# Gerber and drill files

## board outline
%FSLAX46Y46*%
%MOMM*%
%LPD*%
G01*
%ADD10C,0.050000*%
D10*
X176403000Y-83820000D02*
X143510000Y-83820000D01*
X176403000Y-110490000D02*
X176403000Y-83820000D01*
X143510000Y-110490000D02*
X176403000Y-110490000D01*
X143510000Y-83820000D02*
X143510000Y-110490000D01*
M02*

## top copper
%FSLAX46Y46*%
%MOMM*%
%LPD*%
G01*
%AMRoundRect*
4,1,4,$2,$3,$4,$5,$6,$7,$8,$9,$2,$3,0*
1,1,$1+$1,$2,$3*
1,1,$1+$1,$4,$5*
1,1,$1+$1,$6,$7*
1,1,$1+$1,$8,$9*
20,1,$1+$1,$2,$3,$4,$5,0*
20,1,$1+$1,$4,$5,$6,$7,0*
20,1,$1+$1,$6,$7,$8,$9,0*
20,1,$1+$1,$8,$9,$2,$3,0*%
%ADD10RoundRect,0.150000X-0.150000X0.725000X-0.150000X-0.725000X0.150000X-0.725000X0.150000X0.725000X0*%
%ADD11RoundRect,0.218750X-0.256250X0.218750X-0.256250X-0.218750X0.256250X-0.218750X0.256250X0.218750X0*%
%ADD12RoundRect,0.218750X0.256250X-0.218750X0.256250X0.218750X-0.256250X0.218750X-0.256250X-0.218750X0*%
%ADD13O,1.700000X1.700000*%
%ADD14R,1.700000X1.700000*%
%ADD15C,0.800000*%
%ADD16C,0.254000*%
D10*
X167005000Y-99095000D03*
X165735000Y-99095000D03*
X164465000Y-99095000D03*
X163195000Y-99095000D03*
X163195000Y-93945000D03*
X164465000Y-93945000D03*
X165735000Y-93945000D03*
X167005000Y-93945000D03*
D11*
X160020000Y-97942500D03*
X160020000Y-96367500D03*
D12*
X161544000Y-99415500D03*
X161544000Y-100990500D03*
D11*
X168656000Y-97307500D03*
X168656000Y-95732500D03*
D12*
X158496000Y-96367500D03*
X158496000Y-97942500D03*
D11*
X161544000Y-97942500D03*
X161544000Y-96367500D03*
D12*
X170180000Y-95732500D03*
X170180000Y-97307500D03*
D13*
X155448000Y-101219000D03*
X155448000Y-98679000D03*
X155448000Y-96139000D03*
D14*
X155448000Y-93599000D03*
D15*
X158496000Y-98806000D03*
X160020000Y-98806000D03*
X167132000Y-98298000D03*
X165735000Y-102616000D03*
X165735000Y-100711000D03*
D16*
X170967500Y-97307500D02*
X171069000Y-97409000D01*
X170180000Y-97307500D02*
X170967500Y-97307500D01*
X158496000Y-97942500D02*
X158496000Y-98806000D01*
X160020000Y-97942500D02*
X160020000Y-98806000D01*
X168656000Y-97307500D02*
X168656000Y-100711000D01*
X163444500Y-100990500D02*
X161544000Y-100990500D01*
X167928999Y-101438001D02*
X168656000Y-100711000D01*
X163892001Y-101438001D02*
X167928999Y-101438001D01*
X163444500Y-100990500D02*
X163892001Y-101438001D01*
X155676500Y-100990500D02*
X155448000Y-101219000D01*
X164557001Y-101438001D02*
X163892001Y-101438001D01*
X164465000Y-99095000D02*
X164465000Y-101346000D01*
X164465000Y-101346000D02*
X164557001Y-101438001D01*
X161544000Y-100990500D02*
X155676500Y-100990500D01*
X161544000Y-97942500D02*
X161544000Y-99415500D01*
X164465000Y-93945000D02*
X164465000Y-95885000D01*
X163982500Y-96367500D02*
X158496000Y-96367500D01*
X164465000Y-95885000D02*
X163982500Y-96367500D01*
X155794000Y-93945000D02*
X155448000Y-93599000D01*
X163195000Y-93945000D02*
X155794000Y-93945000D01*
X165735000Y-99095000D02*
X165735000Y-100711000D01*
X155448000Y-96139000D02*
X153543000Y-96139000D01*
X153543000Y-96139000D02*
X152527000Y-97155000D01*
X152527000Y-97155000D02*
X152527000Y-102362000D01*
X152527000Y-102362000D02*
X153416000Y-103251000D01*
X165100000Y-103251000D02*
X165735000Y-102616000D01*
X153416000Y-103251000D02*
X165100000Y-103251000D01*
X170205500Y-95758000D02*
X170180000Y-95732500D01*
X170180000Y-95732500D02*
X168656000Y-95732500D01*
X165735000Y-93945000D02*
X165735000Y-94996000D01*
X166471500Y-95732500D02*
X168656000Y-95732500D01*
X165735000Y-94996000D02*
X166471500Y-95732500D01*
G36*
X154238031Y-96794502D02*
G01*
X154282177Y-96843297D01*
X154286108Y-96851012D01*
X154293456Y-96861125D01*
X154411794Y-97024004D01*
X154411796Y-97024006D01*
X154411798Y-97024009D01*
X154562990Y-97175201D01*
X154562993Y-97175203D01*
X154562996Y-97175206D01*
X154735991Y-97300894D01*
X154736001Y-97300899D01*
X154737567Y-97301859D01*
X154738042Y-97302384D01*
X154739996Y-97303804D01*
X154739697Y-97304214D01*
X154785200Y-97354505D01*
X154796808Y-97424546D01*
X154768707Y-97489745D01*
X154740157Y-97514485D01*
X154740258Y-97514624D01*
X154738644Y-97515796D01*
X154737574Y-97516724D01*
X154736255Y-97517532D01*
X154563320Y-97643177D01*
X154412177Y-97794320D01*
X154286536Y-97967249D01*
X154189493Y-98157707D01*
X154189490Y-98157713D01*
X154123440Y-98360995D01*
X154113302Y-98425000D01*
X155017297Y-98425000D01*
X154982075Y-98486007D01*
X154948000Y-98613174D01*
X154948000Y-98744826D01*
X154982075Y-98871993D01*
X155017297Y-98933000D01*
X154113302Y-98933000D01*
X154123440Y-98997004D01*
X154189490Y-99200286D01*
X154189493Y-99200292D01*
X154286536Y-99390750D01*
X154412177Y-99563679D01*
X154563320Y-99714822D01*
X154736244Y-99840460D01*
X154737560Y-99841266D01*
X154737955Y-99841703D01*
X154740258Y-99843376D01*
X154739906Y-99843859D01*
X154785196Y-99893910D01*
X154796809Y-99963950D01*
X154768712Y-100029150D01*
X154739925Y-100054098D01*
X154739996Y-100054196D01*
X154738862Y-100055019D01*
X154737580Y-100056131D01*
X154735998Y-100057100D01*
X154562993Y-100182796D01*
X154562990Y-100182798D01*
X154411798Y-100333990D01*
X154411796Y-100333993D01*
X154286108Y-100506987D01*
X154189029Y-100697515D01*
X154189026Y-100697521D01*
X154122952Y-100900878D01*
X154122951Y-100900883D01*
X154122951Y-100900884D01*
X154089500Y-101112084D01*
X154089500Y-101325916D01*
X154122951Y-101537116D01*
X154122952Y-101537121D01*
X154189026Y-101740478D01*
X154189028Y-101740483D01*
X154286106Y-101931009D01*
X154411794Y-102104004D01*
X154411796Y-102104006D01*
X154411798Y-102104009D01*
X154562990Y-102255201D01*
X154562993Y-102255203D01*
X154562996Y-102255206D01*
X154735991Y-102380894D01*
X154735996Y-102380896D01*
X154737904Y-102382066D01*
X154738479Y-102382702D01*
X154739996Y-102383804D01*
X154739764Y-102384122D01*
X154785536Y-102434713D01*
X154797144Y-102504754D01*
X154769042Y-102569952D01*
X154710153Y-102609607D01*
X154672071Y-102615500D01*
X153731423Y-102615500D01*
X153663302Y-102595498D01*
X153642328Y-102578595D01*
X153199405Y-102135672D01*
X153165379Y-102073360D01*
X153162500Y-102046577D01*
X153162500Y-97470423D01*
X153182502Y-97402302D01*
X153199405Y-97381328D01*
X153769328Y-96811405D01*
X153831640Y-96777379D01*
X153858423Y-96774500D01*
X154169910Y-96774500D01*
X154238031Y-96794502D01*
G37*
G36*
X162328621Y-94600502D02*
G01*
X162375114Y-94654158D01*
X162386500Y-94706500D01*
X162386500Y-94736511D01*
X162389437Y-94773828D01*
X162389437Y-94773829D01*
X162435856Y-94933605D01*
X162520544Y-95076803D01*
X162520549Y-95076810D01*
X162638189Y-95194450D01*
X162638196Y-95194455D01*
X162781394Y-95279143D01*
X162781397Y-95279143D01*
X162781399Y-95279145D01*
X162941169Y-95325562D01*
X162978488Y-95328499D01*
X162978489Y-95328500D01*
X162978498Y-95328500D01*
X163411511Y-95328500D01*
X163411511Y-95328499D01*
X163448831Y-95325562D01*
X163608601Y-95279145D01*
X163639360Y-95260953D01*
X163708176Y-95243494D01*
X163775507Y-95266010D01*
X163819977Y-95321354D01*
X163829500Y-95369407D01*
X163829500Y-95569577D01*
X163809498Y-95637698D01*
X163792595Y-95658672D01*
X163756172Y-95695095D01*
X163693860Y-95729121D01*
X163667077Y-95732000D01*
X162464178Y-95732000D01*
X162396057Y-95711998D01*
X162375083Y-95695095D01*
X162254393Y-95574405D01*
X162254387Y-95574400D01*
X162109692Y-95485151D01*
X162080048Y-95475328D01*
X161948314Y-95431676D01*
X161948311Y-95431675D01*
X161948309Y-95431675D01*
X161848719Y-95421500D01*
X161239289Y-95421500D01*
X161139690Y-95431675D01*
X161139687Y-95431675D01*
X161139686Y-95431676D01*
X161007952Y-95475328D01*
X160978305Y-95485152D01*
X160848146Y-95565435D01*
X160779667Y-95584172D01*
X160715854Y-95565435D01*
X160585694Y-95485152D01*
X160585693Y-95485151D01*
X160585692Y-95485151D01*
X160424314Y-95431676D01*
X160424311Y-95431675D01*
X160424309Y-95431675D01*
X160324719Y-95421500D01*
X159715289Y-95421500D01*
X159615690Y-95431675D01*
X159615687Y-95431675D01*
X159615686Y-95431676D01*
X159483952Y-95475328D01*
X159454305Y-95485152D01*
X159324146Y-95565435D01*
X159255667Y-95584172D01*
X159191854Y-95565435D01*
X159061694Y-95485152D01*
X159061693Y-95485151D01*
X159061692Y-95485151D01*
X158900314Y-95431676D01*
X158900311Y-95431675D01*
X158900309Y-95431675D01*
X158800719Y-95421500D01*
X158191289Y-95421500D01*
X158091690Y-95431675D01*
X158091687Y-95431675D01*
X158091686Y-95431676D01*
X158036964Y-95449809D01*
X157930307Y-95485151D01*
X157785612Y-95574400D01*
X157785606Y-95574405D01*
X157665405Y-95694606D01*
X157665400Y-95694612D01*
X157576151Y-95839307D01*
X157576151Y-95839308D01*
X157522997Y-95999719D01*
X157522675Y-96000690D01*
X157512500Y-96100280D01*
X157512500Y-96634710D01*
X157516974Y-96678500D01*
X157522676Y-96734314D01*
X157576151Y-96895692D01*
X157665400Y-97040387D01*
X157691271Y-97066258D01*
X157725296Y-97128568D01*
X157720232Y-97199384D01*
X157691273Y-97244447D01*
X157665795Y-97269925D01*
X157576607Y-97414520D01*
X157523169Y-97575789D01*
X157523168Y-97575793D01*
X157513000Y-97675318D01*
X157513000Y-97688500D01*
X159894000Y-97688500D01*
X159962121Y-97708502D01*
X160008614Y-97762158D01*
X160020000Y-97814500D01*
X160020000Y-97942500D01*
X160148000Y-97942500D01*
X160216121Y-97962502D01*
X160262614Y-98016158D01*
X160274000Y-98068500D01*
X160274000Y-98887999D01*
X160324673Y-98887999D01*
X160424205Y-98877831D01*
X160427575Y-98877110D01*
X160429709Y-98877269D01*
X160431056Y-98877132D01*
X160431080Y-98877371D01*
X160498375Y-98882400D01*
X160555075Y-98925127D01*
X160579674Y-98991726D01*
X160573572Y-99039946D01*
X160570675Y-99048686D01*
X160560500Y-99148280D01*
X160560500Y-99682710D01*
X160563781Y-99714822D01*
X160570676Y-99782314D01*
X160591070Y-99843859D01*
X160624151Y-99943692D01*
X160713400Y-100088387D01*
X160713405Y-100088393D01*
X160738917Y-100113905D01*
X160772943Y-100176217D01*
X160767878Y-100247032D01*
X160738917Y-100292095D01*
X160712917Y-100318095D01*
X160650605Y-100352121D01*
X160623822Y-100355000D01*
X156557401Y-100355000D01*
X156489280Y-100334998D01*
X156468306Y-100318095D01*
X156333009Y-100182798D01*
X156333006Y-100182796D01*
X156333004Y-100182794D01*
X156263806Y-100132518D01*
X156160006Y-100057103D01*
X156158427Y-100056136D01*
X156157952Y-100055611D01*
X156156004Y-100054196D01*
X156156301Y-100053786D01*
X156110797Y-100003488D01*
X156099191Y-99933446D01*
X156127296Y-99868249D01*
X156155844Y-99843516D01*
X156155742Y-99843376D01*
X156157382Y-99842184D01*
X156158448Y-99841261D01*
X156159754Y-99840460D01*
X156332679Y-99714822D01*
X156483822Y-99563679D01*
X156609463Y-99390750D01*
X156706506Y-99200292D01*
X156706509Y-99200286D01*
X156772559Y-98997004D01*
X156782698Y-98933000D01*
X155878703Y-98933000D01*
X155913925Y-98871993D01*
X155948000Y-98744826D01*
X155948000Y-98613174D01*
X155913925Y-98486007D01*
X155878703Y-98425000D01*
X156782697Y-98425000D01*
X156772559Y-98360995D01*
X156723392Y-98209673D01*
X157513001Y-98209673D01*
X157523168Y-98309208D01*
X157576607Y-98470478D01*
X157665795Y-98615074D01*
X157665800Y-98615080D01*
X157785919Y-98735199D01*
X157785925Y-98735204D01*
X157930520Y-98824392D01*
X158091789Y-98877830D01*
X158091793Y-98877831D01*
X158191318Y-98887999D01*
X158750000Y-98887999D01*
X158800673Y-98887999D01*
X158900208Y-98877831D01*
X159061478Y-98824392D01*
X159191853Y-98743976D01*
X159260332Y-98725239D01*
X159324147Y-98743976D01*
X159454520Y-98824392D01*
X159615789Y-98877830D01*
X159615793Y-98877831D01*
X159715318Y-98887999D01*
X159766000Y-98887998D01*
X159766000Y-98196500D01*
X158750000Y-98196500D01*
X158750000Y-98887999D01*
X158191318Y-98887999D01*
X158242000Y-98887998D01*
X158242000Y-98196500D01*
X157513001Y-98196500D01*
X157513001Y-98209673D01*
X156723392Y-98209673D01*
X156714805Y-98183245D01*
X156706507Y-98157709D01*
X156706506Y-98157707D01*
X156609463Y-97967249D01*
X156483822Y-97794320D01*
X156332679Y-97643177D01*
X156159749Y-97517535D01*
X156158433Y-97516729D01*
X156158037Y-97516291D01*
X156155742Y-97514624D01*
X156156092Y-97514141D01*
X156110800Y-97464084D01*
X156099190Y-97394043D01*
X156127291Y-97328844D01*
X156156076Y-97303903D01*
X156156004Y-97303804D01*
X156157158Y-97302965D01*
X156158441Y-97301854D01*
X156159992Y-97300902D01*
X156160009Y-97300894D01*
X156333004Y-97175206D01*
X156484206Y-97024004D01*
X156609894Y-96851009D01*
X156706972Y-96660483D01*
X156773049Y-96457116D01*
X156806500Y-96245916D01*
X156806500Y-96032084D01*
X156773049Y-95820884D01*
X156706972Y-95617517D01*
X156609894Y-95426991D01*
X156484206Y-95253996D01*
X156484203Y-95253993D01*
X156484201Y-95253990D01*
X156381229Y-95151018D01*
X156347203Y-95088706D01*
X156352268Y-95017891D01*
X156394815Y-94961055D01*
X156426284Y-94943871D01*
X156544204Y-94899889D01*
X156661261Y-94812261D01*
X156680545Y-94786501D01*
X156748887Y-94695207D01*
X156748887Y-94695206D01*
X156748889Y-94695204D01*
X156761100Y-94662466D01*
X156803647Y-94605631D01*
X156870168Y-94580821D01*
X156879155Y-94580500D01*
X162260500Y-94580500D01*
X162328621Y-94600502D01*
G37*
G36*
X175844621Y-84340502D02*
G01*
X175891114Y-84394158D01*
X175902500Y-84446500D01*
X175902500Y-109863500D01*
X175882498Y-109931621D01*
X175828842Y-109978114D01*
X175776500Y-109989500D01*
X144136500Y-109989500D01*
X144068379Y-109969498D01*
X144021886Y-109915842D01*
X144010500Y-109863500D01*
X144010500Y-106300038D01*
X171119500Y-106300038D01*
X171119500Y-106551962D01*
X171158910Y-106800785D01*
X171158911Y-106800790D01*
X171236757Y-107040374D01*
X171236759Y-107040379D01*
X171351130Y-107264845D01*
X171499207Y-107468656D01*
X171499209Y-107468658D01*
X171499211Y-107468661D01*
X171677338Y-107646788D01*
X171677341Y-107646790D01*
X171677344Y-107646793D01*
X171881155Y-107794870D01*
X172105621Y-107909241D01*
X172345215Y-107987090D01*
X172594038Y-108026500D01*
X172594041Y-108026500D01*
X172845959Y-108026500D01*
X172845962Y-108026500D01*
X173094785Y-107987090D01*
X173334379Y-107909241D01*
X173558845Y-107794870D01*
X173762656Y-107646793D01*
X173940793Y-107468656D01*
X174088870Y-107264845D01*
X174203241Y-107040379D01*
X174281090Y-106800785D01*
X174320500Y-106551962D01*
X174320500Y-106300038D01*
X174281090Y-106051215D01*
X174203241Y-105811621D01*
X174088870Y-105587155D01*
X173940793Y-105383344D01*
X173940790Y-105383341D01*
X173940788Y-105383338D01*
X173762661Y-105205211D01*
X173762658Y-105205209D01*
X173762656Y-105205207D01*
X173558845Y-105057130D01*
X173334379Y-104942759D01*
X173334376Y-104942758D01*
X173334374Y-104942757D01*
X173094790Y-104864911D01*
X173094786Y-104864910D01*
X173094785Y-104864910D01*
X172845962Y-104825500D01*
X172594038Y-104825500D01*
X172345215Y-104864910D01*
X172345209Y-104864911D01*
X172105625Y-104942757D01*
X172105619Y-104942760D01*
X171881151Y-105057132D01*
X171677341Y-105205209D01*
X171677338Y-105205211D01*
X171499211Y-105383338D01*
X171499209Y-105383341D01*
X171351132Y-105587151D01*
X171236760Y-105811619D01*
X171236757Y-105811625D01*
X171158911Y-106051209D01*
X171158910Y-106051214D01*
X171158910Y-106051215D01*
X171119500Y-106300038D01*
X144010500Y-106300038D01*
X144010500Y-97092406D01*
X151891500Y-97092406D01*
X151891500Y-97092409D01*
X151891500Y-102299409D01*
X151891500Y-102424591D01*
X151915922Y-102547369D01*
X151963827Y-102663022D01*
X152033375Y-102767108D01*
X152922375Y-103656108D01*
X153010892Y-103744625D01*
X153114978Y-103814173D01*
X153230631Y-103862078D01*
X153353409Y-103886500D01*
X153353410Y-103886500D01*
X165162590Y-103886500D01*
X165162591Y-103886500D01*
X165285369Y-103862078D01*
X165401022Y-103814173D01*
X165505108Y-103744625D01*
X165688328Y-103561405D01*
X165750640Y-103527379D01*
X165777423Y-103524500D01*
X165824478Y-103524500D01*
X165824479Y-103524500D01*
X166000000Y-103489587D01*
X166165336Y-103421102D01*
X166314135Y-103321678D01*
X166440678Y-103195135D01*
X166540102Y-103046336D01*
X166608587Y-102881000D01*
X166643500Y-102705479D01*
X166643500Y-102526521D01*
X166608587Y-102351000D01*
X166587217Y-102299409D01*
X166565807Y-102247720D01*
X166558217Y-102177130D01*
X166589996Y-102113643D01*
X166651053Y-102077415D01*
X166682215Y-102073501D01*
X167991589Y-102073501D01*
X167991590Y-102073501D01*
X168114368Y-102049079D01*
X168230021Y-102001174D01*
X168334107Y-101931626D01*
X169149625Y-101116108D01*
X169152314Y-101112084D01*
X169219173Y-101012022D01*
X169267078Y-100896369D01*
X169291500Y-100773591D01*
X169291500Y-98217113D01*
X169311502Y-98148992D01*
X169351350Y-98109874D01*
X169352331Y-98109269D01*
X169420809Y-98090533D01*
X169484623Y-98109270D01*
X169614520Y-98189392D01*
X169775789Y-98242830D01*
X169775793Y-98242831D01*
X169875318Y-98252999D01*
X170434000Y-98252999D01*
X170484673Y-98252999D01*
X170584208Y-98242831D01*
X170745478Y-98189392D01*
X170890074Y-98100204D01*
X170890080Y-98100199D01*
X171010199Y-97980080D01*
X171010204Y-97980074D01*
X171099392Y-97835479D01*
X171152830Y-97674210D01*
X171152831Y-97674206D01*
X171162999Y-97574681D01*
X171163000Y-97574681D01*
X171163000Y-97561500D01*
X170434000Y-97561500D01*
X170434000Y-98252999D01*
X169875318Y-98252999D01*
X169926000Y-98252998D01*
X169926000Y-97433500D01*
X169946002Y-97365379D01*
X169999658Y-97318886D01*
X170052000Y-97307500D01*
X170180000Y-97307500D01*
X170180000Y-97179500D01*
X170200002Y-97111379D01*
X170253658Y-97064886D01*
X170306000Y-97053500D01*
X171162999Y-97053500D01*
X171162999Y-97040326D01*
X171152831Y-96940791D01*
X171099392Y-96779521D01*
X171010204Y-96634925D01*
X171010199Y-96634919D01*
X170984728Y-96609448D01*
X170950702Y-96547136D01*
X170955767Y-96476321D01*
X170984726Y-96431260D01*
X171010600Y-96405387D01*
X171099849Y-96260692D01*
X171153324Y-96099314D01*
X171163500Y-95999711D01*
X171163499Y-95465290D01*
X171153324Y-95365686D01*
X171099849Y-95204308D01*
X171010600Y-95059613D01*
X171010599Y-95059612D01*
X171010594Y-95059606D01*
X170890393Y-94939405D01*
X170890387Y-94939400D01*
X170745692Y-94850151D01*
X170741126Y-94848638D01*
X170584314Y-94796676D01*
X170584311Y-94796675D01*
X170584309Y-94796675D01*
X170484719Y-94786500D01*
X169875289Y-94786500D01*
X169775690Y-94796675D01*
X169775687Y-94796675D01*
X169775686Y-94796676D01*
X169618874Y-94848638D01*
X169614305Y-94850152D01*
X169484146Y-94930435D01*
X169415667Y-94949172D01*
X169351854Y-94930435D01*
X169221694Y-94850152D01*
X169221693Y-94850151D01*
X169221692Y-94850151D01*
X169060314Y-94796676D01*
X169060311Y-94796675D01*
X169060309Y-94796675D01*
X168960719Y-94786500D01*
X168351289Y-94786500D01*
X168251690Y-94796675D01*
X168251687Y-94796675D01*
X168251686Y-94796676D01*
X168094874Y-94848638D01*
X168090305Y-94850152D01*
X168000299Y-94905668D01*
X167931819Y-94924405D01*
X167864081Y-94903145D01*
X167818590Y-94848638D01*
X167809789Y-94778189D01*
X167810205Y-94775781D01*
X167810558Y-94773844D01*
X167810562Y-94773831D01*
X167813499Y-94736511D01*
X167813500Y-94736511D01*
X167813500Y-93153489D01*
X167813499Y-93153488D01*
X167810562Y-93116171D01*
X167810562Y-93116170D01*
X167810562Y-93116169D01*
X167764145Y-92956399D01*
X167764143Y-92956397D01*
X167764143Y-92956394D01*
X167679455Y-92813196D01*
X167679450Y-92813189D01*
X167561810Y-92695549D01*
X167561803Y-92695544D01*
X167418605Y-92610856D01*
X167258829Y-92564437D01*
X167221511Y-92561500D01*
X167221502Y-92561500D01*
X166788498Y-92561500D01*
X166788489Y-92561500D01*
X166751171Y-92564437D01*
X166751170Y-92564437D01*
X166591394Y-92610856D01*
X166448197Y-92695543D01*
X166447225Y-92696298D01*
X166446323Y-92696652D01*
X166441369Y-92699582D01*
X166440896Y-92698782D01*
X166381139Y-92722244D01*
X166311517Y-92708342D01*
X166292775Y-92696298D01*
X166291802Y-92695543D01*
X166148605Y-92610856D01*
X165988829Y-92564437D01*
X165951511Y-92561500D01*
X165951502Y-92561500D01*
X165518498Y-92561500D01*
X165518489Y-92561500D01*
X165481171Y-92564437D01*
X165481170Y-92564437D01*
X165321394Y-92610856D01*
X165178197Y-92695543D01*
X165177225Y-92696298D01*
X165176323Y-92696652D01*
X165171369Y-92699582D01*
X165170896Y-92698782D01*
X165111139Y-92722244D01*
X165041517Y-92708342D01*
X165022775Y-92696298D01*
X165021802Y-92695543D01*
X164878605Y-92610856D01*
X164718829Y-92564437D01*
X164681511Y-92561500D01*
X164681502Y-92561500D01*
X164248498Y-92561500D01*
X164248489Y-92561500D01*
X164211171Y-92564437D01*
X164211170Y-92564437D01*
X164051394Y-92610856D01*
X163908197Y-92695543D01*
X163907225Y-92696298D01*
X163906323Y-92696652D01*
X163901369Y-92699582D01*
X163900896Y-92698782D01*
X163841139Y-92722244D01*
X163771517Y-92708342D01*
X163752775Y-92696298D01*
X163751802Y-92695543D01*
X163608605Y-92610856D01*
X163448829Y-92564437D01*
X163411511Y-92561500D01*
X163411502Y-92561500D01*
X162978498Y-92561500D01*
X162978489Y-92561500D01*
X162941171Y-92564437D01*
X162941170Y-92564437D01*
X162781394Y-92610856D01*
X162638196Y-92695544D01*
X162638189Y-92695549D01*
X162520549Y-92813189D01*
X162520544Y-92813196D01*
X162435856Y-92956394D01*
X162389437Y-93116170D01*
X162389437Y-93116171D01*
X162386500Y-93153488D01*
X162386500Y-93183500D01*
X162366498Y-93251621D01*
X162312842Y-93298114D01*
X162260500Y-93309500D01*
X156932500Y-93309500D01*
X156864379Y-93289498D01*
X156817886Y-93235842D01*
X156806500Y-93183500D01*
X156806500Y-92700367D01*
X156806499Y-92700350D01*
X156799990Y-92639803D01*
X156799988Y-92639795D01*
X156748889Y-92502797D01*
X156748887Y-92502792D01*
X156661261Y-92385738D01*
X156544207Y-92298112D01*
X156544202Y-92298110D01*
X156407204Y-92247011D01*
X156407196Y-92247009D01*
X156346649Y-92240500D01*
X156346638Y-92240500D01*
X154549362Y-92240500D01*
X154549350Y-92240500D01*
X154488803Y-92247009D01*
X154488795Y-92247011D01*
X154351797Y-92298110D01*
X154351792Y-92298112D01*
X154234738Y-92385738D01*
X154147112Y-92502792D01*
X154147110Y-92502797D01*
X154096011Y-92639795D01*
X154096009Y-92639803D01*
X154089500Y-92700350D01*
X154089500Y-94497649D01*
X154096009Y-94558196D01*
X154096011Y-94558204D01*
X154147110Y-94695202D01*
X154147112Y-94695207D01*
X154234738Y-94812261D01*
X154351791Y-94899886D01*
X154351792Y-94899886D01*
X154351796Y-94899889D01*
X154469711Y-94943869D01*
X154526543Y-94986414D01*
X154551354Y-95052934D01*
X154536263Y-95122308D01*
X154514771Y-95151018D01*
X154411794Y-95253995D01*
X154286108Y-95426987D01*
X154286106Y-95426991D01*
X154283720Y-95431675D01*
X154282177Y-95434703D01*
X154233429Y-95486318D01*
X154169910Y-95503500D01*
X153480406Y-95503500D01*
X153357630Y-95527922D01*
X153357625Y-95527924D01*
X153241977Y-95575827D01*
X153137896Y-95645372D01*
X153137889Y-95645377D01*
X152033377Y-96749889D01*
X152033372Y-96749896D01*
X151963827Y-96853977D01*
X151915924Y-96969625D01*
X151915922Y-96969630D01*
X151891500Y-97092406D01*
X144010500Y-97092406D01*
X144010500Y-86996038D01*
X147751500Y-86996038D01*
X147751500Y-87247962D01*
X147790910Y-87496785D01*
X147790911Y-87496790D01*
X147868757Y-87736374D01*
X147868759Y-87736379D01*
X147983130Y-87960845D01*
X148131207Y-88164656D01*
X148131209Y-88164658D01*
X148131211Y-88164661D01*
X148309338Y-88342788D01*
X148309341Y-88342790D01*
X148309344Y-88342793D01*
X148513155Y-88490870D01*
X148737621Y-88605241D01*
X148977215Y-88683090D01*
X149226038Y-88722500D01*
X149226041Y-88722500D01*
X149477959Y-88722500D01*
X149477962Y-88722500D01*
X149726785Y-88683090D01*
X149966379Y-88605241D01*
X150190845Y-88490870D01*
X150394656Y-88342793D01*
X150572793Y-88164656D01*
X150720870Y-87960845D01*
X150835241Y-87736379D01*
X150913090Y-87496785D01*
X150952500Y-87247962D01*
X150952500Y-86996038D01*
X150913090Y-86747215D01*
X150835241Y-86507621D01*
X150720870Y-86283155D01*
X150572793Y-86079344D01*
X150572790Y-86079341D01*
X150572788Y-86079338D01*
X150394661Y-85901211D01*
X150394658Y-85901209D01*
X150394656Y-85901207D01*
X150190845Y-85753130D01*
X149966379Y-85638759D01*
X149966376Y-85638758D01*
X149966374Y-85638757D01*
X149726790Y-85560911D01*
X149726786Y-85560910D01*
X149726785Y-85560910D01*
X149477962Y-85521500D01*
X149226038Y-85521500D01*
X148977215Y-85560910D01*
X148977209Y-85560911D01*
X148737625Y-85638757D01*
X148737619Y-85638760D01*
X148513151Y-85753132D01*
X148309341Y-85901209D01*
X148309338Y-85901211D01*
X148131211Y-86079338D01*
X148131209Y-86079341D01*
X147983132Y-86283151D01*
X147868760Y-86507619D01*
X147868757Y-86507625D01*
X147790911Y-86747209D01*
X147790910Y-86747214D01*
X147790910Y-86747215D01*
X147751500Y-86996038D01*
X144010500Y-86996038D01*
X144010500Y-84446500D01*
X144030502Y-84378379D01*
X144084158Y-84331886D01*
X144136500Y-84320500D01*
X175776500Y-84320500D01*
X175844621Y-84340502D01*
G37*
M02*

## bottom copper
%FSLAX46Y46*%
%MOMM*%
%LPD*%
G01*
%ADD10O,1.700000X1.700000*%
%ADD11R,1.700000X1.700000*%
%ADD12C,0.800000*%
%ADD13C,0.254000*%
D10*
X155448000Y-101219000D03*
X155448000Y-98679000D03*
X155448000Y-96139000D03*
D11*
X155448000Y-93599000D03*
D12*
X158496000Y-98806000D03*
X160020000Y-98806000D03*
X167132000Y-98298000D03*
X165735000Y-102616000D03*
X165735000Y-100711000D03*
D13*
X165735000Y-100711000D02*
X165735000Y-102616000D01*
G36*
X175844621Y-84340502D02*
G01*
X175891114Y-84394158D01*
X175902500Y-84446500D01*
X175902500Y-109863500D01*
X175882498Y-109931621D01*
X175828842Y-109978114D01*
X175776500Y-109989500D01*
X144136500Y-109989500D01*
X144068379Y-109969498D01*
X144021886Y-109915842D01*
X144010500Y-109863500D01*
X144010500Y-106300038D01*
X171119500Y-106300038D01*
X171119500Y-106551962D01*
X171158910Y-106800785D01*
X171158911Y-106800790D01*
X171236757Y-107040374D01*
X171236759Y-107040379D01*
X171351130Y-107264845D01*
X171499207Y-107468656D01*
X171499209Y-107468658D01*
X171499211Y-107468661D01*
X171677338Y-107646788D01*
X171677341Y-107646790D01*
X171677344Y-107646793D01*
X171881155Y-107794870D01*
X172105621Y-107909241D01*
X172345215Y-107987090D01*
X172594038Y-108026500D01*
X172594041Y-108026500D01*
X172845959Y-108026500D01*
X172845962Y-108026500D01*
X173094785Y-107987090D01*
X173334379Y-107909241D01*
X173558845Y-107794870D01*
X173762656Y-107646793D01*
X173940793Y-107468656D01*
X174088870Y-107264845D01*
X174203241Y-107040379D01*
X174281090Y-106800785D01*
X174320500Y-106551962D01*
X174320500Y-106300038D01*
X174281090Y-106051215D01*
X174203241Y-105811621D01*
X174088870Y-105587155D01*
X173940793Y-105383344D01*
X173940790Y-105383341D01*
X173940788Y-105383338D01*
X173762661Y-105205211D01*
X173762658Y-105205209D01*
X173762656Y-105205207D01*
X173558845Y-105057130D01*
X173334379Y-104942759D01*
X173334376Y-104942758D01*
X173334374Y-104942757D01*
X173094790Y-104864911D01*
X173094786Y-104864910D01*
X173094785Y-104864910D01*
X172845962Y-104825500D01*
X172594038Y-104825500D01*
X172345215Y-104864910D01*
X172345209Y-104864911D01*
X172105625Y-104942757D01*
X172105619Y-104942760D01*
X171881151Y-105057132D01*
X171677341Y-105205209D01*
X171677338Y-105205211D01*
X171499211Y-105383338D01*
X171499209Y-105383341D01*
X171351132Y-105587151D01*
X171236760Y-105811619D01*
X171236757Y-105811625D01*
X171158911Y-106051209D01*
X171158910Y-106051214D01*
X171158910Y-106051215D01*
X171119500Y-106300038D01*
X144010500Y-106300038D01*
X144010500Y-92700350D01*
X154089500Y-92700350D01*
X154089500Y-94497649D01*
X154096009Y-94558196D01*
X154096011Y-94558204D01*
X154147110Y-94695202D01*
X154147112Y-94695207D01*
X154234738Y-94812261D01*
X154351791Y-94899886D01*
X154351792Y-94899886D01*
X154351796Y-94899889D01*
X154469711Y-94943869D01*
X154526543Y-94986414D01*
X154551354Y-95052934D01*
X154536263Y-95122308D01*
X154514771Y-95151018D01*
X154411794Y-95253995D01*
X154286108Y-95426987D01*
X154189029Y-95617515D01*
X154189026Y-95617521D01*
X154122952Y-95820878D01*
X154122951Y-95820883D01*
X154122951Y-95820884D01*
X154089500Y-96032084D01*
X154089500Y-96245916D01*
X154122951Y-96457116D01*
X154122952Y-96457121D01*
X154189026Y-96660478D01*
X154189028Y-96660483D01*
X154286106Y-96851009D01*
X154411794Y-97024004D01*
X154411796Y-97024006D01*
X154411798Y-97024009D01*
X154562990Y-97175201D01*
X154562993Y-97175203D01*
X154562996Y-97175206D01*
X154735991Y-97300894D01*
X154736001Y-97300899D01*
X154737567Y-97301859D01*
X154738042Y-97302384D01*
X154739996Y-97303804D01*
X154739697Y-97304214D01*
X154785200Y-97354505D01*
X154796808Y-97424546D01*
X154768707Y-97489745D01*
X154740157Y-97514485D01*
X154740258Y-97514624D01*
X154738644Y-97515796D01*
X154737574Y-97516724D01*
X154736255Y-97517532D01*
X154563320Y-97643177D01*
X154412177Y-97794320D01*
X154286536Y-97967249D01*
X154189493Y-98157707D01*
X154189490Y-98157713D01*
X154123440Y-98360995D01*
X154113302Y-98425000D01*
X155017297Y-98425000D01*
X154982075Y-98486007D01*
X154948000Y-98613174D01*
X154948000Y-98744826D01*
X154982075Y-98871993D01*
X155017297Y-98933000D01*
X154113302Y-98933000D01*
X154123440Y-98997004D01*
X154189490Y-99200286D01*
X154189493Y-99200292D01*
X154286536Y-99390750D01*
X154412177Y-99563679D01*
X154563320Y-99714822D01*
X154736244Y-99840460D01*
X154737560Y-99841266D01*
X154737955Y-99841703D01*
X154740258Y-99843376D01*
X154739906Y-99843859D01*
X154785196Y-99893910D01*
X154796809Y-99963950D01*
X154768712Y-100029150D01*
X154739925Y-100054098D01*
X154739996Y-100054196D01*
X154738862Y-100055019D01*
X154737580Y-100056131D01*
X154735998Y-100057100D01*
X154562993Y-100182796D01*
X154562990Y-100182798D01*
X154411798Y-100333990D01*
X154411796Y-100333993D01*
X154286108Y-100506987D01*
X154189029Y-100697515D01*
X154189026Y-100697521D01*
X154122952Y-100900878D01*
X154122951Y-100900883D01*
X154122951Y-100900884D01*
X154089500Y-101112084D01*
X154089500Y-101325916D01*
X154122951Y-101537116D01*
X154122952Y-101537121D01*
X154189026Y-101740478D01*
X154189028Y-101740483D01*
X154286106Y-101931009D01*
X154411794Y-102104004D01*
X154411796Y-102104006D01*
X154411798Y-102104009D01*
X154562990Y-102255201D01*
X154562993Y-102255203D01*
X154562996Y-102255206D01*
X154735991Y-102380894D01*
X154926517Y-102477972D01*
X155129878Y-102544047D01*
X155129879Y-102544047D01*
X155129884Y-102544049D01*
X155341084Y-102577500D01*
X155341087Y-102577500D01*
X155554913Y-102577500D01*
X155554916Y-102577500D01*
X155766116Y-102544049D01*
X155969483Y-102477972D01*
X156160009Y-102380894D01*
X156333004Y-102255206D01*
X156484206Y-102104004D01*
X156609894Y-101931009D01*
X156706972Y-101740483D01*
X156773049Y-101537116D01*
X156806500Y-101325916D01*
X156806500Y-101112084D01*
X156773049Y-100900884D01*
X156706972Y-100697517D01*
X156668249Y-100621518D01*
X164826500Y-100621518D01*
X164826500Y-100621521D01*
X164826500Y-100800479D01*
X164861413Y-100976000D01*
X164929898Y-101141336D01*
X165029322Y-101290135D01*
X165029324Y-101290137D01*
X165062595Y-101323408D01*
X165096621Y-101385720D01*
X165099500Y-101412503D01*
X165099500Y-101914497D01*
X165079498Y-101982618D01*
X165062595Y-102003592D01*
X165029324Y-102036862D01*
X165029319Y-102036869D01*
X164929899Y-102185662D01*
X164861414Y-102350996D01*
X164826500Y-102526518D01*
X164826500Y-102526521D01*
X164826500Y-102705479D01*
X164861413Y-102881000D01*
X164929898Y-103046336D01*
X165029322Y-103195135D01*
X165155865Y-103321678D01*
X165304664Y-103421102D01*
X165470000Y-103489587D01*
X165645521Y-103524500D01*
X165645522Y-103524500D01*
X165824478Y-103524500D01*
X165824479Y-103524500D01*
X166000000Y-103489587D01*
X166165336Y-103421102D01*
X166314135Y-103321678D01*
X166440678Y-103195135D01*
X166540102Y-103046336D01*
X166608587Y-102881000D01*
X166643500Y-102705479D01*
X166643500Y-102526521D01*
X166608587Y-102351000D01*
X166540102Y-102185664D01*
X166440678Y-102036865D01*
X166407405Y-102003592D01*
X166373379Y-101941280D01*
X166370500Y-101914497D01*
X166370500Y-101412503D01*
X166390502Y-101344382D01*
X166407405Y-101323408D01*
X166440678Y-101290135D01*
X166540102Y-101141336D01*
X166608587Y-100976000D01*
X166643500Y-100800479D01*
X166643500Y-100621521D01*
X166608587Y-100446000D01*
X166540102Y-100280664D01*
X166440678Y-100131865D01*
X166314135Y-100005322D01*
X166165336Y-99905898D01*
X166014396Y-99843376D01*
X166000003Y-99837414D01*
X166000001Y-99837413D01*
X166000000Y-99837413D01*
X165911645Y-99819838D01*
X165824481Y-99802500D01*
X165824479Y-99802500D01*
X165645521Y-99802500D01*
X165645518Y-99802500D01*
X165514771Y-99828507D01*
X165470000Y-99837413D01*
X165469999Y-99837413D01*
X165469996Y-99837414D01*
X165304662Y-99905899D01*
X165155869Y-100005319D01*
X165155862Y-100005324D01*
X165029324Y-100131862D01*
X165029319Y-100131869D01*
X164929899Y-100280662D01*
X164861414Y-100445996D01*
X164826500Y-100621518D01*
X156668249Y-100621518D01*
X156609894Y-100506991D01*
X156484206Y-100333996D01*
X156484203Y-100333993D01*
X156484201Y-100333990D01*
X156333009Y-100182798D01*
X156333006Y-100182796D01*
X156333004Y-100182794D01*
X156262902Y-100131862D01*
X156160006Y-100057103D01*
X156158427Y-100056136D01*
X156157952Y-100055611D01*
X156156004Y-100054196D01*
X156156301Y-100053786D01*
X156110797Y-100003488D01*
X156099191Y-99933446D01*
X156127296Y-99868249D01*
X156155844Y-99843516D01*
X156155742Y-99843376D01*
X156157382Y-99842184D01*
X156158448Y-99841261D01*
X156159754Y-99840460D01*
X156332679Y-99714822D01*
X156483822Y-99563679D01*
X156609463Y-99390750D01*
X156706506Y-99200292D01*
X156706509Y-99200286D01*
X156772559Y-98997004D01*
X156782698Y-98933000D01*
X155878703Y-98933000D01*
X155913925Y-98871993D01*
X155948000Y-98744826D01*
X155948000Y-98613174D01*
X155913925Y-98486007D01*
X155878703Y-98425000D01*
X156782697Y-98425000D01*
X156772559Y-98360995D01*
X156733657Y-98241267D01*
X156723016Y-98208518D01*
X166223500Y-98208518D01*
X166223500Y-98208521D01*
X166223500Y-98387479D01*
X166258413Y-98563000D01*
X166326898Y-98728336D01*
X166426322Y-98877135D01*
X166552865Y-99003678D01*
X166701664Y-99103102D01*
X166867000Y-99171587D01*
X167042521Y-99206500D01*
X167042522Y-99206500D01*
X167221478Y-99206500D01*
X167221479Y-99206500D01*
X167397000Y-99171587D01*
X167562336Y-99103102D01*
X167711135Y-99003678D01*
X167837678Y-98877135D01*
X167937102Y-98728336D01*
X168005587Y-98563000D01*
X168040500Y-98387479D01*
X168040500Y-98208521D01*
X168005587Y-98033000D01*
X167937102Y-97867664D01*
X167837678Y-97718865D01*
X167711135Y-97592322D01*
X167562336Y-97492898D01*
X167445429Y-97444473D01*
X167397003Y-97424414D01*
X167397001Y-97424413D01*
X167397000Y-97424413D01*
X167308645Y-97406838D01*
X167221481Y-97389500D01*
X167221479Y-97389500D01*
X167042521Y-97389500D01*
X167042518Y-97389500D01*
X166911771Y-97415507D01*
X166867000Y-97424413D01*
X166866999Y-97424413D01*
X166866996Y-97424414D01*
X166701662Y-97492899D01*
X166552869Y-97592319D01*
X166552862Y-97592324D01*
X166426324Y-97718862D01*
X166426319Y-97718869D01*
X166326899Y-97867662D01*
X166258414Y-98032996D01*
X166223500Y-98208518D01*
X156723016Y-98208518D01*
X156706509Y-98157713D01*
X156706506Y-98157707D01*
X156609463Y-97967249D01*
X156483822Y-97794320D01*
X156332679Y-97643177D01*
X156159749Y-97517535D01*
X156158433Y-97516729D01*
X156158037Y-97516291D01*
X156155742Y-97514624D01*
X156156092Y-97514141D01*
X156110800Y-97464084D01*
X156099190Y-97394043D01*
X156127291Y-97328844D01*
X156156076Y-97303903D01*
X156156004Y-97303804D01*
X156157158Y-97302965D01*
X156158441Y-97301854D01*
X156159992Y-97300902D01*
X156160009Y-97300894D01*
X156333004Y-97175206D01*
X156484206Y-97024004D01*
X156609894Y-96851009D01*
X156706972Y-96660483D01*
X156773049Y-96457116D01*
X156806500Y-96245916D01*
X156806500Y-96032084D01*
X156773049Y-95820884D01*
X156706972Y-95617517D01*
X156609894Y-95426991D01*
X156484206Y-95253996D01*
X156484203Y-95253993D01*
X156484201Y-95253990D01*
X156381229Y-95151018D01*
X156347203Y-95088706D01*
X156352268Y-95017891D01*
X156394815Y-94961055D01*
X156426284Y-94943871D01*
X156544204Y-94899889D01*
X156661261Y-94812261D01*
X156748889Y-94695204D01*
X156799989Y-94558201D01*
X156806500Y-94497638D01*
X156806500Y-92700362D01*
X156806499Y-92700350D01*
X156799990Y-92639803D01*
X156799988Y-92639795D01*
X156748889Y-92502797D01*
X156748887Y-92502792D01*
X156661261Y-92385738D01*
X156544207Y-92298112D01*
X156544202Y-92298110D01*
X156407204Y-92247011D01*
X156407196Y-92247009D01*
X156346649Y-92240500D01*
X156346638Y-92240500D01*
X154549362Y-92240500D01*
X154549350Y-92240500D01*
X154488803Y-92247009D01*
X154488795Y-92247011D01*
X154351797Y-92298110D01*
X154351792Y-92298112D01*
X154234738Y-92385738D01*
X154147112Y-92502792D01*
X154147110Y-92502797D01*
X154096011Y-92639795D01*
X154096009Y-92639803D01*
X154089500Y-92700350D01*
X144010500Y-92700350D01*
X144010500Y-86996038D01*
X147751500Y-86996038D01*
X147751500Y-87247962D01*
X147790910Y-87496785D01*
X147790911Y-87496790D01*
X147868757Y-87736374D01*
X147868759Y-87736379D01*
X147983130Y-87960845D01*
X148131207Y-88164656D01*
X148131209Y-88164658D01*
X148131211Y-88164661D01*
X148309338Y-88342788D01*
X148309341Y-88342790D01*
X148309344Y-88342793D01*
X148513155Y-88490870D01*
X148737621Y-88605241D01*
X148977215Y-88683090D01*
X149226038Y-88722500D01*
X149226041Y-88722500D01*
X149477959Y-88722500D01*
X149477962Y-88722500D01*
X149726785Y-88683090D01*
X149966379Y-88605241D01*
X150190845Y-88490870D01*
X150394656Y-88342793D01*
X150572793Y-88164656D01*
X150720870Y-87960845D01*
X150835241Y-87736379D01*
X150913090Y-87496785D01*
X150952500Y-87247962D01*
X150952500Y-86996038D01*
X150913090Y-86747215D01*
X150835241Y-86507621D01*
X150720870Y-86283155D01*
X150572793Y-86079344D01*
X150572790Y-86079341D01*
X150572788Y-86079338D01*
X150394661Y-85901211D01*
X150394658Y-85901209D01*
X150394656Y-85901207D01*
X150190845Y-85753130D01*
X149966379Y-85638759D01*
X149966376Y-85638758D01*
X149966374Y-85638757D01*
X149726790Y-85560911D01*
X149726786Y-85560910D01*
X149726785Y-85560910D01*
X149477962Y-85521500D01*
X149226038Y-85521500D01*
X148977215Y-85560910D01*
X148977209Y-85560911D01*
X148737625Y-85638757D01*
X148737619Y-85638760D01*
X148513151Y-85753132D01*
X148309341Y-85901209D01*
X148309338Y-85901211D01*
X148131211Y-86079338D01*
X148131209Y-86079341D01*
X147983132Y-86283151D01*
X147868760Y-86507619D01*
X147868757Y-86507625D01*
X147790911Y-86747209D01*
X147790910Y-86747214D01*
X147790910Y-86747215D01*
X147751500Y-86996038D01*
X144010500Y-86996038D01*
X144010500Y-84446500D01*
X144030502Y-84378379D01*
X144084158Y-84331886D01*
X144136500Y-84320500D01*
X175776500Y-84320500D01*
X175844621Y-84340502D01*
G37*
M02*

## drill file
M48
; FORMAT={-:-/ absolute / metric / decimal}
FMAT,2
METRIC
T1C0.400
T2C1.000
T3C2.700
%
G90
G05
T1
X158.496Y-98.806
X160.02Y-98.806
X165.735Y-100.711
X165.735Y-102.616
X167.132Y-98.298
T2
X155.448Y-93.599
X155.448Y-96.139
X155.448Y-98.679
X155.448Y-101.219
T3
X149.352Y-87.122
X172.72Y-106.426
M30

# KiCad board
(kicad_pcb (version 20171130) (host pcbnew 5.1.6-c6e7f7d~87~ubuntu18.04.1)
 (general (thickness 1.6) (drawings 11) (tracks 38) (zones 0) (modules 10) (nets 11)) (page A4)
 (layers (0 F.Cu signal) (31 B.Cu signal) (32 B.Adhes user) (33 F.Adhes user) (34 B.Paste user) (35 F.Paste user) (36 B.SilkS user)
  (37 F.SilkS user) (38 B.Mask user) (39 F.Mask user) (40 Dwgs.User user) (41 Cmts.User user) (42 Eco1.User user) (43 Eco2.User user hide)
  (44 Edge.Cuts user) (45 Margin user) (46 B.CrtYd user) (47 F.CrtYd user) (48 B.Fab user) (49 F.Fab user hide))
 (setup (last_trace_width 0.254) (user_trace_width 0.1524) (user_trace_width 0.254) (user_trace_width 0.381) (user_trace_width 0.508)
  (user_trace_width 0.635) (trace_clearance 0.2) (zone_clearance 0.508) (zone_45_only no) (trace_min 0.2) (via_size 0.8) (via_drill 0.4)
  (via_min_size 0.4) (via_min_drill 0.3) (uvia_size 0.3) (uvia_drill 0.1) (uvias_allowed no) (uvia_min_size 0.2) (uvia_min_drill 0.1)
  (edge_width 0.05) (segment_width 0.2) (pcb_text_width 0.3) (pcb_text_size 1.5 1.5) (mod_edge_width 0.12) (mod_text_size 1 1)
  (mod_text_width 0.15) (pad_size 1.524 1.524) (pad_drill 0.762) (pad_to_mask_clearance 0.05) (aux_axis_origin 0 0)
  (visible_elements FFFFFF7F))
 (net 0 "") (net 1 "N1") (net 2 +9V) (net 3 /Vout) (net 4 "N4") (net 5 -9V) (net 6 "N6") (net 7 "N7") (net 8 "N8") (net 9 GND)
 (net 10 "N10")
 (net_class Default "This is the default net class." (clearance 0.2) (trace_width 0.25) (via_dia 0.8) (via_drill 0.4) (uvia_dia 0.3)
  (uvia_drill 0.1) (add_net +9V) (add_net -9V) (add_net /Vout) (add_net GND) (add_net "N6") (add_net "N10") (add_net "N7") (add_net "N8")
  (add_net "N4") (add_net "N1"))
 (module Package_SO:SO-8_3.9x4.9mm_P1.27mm (layer F.Cu) (at 165.1 96.52 270)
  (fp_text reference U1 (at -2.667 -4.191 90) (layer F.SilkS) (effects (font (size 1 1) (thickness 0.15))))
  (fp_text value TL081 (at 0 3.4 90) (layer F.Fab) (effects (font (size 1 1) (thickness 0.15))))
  (pad 8 smd roundrect (at 2.575 -1.905 270) (size 1.75 0.6) (layers F.Cu F.Paste F.Mask) (roundrect_rratio 0.25) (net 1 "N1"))
  (pad 7 smd roundrect (at 2.575 -0.635 270) (size 1.75 0.6) (layers F.Cu F.Paste F.Mask) (roundrect_rratio 0.25) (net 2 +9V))
  (pad 6 smd roundrect (at 2.575 0.635 270) (size 1.75 0.6) (layers F.Cu F.Paste F.Mask) (roundrect_rratio 0.25) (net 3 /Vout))
  (pad 5 smd roundrect (at 2.575 1.905 270) (size 1.75 0.6) (layers F.Cu F.Paste F.Mask) (roundrect_rratio 0.25) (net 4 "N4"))
  (pad 4 smd roundrect (at -2.575 1.905 270) (size 1.75 0.6) (layers F.Cu F.Paste F.Mask) (roundrect_rratio 0.25) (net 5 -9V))
  (pad 3 smd roundrect (at -2.575 0.635 270) (size 1.75 0.6) (layers F.Cu F.Paste F.Mask) (roundrect_rratio 0.25) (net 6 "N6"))
  (pad 2 smd roundrect (at -2.575 -0.635 270) (size 1.75 0.6) (layers F.Cu F.Paste F.Mask) (roundrect_rratio 0.25) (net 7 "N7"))
  (pad 1 smd roundrect (at -2.575 -1.905 270) (size 1.75 0.6) (layers F.Cu F.Paste F.Mask) (roundrect_rratio 0.25) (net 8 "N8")))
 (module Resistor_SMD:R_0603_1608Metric (layer F.Cu) (at 160.02 97.155 270)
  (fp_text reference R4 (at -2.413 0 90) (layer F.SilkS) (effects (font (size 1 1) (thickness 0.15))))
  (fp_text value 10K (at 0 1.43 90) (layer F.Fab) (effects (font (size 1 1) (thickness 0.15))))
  (pad 2 smd roundrect (at 0.7875 0 270) (size 0.875 0.95) (layers F.Cu F.Paste F.Mask) (roundrect_rratio 0.25) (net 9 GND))
  (pad 1 smd roundrect (at -0.7875 0 270) (size 0.875 0.95) (layers F.Cu F.Paste F.Mask) (roundrect_rratio 0.25) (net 6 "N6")))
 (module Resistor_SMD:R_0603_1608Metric (layer F.Cu) (at 161.544 100.203 90)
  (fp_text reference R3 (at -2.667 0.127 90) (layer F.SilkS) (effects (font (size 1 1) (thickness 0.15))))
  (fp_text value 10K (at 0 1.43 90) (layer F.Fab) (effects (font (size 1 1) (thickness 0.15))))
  (pad 2 smd roundrect (at 0.7875 0 90) (size 0.875 0.95) (layers F.Cu F.Paste F.Mask) (roundrect_rratio 0.25) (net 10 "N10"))
  (pad 1 smd roundrect (at -0.7875 0 90) (size 0.875 0.95) (layers F.Cu F.Paste F.Mask) (roundrect_rratio 0.25) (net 3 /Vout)))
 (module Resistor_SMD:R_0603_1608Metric (layer F.Cu) (at 168.656 96.52 270)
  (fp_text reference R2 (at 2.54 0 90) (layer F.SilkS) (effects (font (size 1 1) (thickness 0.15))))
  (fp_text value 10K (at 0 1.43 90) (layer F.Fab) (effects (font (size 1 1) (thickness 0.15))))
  (pad 2 smd roundrect (at 0.7875 0 270) (size 0.875 0.95) (layers F.Cu F.Paste F.Mask) (roundrect_rratio 0.25) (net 3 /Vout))
  (pad 1 smd roundrect (at -0.7875 0 270) (size 0.875 0.95) (layers F.Cu F.Paste F.Mask) (roundrect_rratio 0.25) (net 7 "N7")))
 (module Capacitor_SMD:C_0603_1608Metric (layer F.Cu) (at 158.496 97.155 90)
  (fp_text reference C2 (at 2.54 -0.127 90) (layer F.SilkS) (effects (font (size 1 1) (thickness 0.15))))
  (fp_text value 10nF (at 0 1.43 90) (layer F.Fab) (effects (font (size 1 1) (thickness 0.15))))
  (pad 2 smd roundrect (at 0.7875 0 90) (size 0.875 0.95) (layers F.Cu F.Paste F.Mask) (roundrect_rratio 0.25) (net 6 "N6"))
  (pad 1 smd roundrect (at -0.7875 0 90) (size 0.875 0.95) (layers F.Cu F.Paste F.Mask) (roundrect_rratio 0.25) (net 9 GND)))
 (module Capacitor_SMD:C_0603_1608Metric (layer F.Cu) (at 161.544 97.155 270)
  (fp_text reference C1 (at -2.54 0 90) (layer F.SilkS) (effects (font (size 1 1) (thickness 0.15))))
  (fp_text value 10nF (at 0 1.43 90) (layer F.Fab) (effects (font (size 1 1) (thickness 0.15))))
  (pad 2 smd roundrect (at 0.7875 0 270) (size 0.875 0.95) (layers F.Cu F.Paste F.Mask) (roundrect_rratio 0.25) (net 10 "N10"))
  (pad 1 smd roundrect (at -0.7875 0 270) (size 0.875 0.95) (layers F.Cu F.Paste F.Mask) (roundrect_rratio 0.25) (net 6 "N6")))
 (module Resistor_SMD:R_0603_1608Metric (layer F.Cu) (at 170.18 96.52 90)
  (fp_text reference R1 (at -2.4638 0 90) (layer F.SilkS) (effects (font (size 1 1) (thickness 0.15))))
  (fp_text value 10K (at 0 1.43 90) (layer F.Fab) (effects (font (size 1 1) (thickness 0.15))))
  (pad 2 smd roundrect (at 0.7875 0 90) (size 0.875 0.95) (layers F.Cu F.Paste F.Mask) (roundrect_rratio 0.25) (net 7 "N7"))
  (pad 1 smd roundrect (at -0.7875 0 90) (size 0.875 0.95) (layers F.Cu F.Paste F.Mask) (roundrect_rratio 0.25) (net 9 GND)))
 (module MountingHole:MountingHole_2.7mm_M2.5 (layer F.Cu) (at 172.72 106.426)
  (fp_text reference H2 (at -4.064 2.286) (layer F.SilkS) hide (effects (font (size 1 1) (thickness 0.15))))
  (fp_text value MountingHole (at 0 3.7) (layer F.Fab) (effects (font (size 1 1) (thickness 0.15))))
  (pad 1 np_thru_hole circle (at 0 0) (size 2.7 2.7) (drill 2.7) (layers *.Cu *.Mask)))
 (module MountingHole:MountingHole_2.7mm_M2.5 (layer F.Cu) (at 149.352 87.122)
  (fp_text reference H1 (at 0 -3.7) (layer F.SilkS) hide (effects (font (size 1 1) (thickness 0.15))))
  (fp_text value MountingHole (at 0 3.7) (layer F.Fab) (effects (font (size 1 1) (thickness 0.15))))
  (pad 1 np_thru_hole circle (at 0 0) (size 2.7 2.7) (drill 2.7) (layers *.Cu *.Mask)))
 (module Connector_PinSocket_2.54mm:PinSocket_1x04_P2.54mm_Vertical (layer F.Cu) (at 155.448 93.599)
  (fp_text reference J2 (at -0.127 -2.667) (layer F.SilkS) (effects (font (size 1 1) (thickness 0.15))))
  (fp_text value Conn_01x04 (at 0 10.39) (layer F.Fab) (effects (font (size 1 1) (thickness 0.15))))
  (pad 4 thru_hole oval (at 0 7.62) (size 1.7 1.7) (drill 1) (layers *.Cu *.Mask) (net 3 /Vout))
  (pad 3 thru_hole oval (at 0 5.08) (size 1.7 1.7) (drill 1) (layers *.Cu *.Mask) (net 9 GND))
  (pad 2 thru_hole oval (at 0 2.54) (size 1.7 1.7) (drill 1) (layers *.Cu *.Mask) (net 2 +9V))
  (pad 1 thru_hole rect (at 0 0) (size 1.7 1.7) (drill 1) (layers *.Cu *.Mask) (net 5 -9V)))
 (gr_line (start 176.403 83.82) (end 143.51 83.82) (layer Edge.Cuts) (width 0.05))
 (gr_line (start 176.403 110.49) (end 176.403 83.82) (layer Edge.Cuts) (width 0.05))
 (gr_line (start 143.51 110.49) (end 176.403 110.49) (layer Edge.Cuts) (width 0.05))
 (gr_line (start 143.51 83.82) (end 143.51 110.49) (layer Edge.Cuts) (width 0.05))
 (via (at 158.496 98.806) (size 0.8) (drill 0.4) (layers F.Cu B.Cu) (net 9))
 (via (at 160.02 98.806) (size 0.8) (drill 0.4) (layers F.Cu B.Cu) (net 9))
 (via (at 167.132 98.298) (size 0.8) (drill 0.4) (layers F.Cu B.Cu) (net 1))
 (segment (start 170.9675 97.3075) (end 171.069 97.409) (width 0.254) (layer F.Cu) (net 9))
 (segment (start 170.18 97.3075) (end 170.9675 97.3075) (width 0.254) (layer F.Cu) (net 9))
 (segment (start 158.496 97.9425) (end 158.496 98.806) (width 0.254) (layer F.Cu) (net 9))
 (segment (start 160.02 97.9425) (end 160.02 98.806) (width 0.254) (layer F.Cu) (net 9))
 (segment (start 168.656 97.3075) (end 168.656 100.711) (width 0.254) (layer F.Cu) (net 3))
 (segment (start 163.4445 100.9905) (end 161.544 100.9905) (width 0.254) (layer F.Cu) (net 3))
 (segment (start 167.928999 101.438001) (end 168.656 100.711) (width 0.254) (layer F.Cu) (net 3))
 (segment (start 163.892001 101.438001) (end 167.928999 101.438001) (width 0.254) (layer F.Cu) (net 3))
 (segment (start 163.4445 100.9905) (end 163.892001 101.438001) (width 0.254) (layer F.Cu) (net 3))
 (segment (start 155.6765 100.9905) (end 155.448 101.219) (width 0.254) (layer F.Cu) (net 3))
 (segment (start 164.557001 101.438001) (end 163.892001 101.438001) (width 0.254) (layer F.Cu) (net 3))
 (segment (start 164.465 99.095) (end 164.465 101.346) (width 0.254) (layer F.Cu) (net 3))
 (segment (start 164.465 101.346) (end 164.557001 101.438001) (width 0.254) (layer F.Cu) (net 3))
 (segment (start 161.544 100.9905) (end 155.6765 100.9905) (width 0.254) (layer F.Cu) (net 3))
 (segment (start 161.544 97.9425) (end 161.544 99.4155) (width 0.254) (layer F.Cu) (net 10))
 (segment (start 164.465 93.945) (end 164.465 95.885) (width 0.254) (layer F.Cu) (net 6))
 (segment (start 163.9825 96.3675) (end 158.496 96.3675) (width 0.254) (layer F.Cu) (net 6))
 (segment (start 164.465 95.885) (end 163.9825 96.3675) (width 0.254) (layer F.Cu) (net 6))
 (segment (start 155.794 93.945) (end 155.448 93.599) (width 0.254) (layer F.Cu) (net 5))
 (segment (start 163.195 93.945) (end 155.794 93.945) (width 0.254) (layer F.Cu) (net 5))
 (via (at 165.735 102.616) (size 0.8) (drill 0.4) (layers F.Cu B.Cu) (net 2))
 (via (at 165.735 100.711) (size 0.8) (drill 0.4) (layers F.Cu B.Cu) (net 2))
 (segment (start 165.735 99.095) (end 165.735 100.711) (width 0.254) (layer F.Cu) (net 2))
 (segment (start 155.448 96.139) (end 153.543 96.139) (width 0.254) (layer F.Cu) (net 2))
 (segment (start 153.543 96.139) (end 152.527 97.155) (width 0.254) (layer F.Cu) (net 2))
 (segment (start 152.527 97.155) (end 152.527 102.362) (width 0.254) (layer F.Cu) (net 2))
 (segment (start 152.527 102.362) (end 153.416 103.251) (width 0.254) (layer F.Cu) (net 2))
 (segment (start 165.735 100.711) (end 165.735 102.616) (width 0.254) (layer B.Cu) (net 2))
 (segment (start 165.1 103.251) (end 165.735 102.616) (width 0.254) (layer F.Cu) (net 2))
 (segment (start 153.416 103.251) (end 165.1 103.251) (width 0.254) (layer F.Cu) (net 2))
 (segment (start 170.2055 95.758) (end 170.18 95.7325) (width 0.254) (layer F.Cu) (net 7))
 (segment (start 170.18 95.7325) (end 168.656 95.7325) (width 0.254) (layer F.Cu) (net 7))
 (segment (start 165.735 93.945) (end 165.735 94.996) (width 0.254) (layer F.Cu) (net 7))
 (segment (start 166.4715 95.7325) (end 168.656 95.7325) (width 0.254) (layer F.Cu) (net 7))
 (segment (start 165.735 94.996) (end 166.4715 95.7325) (width 0.254) (layer F.Cu) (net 7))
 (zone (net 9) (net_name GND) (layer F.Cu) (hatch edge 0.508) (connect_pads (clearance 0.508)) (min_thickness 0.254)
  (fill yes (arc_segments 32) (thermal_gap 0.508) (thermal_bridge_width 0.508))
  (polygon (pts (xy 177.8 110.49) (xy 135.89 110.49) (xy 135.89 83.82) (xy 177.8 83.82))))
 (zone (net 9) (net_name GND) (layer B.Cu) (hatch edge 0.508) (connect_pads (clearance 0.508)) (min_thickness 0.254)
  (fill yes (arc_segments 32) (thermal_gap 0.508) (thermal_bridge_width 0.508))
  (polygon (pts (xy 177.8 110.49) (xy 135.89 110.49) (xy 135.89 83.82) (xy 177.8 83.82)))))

